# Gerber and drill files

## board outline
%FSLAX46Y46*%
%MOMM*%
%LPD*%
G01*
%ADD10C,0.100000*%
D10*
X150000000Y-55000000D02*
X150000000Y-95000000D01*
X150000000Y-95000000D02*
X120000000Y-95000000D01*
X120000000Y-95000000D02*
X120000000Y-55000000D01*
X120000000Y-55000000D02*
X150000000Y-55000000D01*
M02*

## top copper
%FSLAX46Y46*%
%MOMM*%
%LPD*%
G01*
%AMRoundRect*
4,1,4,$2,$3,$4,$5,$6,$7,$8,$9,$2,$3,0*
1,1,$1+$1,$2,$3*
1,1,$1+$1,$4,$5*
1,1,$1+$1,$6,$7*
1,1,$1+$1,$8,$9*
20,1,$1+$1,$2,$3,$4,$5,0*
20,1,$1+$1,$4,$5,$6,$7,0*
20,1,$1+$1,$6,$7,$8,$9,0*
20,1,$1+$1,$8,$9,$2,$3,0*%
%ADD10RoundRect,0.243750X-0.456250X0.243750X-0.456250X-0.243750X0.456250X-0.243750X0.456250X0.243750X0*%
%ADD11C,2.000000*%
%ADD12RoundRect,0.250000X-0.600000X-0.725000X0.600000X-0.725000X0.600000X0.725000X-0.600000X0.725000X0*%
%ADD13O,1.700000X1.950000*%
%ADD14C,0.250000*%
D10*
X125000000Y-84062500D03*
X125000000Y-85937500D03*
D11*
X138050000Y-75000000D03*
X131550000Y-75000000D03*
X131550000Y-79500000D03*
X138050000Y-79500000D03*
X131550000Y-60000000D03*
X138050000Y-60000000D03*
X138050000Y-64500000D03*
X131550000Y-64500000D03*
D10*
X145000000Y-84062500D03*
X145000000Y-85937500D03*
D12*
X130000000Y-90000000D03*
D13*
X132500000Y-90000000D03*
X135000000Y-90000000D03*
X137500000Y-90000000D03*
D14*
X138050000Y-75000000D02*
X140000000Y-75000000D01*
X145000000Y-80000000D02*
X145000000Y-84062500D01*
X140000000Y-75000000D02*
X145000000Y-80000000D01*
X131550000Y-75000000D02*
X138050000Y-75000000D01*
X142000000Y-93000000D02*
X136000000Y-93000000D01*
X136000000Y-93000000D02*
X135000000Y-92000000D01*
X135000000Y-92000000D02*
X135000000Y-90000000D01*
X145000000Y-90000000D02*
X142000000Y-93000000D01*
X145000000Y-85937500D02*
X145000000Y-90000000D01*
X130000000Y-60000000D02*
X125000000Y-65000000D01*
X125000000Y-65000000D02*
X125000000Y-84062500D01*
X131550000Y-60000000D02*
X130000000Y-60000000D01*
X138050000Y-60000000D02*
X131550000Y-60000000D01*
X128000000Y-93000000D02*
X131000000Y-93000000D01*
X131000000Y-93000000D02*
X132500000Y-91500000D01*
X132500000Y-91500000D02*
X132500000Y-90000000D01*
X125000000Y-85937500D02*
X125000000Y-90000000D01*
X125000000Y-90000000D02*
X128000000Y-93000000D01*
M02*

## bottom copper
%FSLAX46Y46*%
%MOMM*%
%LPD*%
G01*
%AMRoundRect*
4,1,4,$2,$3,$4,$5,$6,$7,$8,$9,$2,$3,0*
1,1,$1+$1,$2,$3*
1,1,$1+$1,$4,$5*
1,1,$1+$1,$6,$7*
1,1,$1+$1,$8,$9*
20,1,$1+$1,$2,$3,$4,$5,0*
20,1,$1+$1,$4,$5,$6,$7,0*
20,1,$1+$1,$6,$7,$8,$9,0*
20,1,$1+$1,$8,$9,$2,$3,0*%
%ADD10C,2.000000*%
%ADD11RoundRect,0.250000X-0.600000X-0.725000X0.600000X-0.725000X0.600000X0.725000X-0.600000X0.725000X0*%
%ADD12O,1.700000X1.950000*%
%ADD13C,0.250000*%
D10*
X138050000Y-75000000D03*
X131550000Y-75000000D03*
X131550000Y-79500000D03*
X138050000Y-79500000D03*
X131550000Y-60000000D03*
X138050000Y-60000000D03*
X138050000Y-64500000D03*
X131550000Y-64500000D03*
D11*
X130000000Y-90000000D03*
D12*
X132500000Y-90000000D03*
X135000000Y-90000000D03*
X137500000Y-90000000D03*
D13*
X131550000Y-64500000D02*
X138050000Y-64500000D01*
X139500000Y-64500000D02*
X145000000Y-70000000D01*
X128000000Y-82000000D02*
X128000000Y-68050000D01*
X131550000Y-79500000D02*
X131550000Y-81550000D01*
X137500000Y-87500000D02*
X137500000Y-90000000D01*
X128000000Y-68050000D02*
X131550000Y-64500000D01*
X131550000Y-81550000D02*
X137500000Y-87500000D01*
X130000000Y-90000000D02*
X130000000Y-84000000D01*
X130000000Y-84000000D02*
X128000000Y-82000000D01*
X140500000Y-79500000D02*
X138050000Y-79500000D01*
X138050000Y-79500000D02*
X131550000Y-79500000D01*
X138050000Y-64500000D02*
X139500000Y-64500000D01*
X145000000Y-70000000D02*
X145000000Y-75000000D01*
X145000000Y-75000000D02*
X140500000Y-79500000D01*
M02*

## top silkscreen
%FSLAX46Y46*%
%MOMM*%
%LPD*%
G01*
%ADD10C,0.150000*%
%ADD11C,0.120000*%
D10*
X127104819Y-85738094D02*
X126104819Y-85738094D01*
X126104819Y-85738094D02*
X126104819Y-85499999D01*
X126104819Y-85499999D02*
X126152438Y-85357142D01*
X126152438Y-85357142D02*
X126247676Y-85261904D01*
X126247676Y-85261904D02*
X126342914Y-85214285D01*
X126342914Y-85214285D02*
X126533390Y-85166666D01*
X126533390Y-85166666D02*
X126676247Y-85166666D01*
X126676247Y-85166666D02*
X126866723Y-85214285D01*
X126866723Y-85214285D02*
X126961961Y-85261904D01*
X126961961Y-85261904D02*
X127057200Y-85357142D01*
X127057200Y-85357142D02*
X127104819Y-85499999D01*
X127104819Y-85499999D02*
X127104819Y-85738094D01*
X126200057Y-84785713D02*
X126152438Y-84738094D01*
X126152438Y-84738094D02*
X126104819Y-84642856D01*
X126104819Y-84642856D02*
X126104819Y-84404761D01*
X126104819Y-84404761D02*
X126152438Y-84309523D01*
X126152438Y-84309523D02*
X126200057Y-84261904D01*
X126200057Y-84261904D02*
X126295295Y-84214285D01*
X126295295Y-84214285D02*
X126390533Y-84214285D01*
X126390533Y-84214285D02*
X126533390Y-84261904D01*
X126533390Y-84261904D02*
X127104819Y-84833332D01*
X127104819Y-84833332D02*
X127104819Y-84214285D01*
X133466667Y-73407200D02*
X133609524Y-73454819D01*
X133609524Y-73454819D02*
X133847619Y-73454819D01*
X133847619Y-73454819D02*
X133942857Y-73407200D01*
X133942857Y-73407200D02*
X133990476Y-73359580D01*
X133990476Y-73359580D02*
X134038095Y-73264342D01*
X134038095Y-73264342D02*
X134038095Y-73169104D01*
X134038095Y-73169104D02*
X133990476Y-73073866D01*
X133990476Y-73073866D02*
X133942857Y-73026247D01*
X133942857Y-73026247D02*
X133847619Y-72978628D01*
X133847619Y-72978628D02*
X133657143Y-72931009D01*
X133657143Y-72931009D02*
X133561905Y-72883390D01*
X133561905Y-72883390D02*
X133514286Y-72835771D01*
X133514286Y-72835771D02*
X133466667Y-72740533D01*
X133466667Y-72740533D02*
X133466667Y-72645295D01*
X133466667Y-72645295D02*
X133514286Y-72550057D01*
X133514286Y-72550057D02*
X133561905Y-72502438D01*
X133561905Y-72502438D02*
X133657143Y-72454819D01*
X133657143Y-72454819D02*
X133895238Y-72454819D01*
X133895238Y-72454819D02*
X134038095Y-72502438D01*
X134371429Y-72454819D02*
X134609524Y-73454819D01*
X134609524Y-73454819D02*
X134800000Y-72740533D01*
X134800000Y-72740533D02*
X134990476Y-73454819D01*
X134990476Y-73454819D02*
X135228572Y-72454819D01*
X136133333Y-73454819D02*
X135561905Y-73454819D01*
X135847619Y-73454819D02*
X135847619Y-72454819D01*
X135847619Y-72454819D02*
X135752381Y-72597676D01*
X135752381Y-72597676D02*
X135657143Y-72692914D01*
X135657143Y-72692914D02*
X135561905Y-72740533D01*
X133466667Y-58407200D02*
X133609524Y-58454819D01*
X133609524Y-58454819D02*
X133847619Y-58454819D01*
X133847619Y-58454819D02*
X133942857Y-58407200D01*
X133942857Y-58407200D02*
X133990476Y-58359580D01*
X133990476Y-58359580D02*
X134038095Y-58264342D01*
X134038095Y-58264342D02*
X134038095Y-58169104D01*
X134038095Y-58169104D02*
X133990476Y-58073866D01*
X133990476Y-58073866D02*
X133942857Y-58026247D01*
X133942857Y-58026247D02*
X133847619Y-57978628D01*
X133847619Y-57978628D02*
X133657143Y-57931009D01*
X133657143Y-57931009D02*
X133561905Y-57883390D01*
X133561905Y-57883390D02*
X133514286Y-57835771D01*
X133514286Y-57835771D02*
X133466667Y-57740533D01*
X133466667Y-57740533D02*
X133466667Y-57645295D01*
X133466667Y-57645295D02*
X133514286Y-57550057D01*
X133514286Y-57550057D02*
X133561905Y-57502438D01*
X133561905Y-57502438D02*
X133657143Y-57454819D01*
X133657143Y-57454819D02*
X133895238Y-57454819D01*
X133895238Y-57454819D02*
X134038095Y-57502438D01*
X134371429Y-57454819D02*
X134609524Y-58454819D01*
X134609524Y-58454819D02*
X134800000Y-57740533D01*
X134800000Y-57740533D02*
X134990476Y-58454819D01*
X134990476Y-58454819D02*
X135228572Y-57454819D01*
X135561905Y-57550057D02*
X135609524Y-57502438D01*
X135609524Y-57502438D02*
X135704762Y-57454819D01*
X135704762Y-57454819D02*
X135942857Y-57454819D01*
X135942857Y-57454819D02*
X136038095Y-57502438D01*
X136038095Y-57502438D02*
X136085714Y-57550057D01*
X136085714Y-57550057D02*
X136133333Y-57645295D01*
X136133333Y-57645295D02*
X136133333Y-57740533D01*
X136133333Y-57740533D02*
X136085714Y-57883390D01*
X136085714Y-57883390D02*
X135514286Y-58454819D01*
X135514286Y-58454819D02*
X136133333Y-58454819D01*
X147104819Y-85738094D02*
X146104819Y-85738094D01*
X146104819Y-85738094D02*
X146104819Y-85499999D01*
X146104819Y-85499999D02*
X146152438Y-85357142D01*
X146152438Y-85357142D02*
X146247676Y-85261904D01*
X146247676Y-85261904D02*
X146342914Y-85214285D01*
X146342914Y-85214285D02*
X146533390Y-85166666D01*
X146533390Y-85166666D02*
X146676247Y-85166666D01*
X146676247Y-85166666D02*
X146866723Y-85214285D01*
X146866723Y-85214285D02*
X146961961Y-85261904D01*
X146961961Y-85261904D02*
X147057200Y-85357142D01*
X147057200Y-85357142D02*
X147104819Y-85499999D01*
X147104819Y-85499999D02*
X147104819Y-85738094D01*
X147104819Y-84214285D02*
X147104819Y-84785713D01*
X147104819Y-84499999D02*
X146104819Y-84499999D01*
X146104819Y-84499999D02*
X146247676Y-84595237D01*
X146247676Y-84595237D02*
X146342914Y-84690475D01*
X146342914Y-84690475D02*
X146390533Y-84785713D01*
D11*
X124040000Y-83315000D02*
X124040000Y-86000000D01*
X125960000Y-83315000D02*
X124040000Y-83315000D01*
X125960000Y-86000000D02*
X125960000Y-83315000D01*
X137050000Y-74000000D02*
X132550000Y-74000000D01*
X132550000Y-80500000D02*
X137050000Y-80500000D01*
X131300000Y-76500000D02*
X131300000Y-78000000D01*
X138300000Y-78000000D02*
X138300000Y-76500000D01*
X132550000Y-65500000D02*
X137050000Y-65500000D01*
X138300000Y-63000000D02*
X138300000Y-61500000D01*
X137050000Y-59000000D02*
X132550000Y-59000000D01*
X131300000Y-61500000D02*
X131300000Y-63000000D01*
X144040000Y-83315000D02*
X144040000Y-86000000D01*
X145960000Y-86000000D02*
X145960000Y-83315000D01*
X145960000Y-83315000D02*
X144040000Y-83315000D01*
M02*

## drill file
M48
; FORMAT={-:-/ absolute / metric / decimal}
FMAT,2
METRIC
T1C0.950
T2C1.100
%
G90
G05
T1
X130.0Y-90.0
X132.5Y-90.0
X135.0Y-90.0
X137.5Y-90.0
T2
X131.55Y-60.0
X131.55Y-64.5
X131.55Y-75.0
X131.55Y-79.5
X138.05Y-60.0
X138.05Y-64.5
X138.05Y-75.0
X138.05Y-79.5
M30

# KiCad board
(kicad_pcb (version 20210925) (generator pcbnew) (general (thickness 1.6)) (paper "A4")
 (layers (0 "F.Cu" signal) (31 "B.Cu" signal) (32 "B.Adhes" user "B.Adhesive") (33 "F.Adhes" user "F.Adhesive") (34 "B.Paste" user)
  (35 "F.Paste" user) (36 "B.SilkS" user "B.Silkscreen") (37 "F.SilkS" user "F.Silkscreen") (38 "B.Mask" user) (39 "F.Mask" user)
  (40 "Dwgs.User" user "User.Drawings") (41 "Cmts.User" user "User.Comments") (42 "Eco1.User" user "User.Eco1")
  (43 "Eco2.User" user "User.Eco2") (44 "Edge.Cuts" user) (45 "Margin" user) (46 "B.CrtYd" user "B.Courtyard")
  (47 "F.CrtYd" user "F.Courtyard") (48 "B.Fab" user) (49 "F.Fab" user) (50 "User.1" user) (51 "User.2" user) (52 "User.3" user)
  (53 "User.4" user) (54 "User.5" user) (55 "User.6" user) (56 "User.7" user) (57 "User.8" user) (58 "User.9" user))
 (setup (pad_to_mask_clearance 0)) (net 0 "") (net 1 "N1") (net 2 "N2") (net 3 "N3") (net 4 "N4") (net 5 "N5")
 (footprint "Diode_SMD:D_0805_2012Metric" (layer "F.Cu") (at 125 85 -90)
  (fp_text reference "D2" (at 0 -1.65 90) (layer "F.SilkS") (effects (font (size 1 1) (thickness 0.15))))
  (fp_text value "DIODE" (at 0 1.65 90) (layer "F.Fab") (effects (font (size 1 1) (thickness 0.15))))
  (fp_line (start -1.685 0.96) (end 1 0.96) (layer "F.SilkS") (width 0.12))
  (fp_line (start -1.685 -0.96) (end -1.685 0.96) (layer "F.SilkS") (width 0.12))
  (fp_line (start 1 -0.96) (end -1.685 -0.96) (layer "F.SilkS") (width 0.12))
  (pad "1" smd roundrect locked (at -0.9375 0 270) (size 0.975 1.4) (layers "F.Cu" "F.Paste" "F.Mask") (roundrect_rratio 0.25) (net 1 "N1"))
  (pad "2" smd roundrect locked (at 0.9375 0 270) (size 0.975 1.4) (layers "F.Cu" "F.Paste" "F.Mask") (roundrect_rratio 0.25) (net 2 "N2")))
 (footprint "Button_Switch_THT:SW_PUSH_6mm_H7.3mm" (layer "F.Cu") (at 131.55 75)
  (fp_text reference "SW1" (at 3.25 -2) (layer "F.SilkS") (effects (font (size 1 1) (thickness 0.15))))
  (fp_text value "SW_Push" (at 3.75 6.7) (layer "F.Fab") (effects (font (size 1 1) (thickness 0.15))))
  (fp_line (start 5.5 -1) (end 1 -1) (layer "F.SilkS") (width 0.12))
  (fp_line (start 1 5.5) (end 5.5 5.5) (layer "F.SilkS") (width 0.12))
  (fp_line (start -0.25 1.5) (end -0.25 3) (layer "F.SilkS") (width 0.12))
  (fp_line (start 6.75 3) (end 6.75 1.5) (layer "F.SilkS") (width 0.12))
  (pad "1" thru_hole circle locked (at 6.5 0 90) (size 2 2) (drill 1.1) (layers *.Cu *.Mask) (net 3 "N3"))
  (pad "1" thru_hole circle locked (at 0 0 90) (size 2 2) (drill 1.1) (layers *.Cu *.Mask) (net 3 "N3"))
  (pad "2" thru_hole circle locked (at 0 4.5 90) (size 2 2) (drill 1.1) (layers *.Cu *.Mask) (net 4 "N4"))
  (pad "2" thru_hole circle locked (at 6.5 4.5 90) (size 2 2) (drill 1.1) (layers *.Cu *.Mask) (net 4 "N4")))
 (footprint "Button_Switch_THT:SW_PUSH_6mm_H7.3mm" (layer "F.Cu") (at 131.55 60)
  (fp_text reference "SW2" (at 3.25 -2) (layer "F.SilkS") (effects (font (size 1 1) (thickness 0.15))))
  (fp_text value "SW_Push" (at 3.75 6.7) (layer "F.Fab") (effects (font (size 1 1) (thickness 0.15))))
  (fp_line (start 1 5.5) (end 5.5 5.5) (layer "F.SilkS") (width 0.12))
  (fp_line (start 6.75 3) (end 6.75 1.5) (layer "F.SilkS") (width 0.12))
  (fp_line (start 5.5 -1) (end 1 -1) (layer "F.SilkS") (width 0.12))
  (fp_line (start -0.25 1.5) (end -0.25 3) (layer "F.SilkS") (width 0.12))
  (pad "1" thru_hole circle locked (at 0 0 90) (size 2 2) (drill 1.1) (layers *.Cu *.Mask) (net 1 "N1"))
  (pad "1" thru_hole circle locked (at 6.5 0 90) (size 2 2) (drill 1.1) (layers *.Cu *.Mask) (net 1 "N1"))
  (pad "2" thru_hole circle locked (at 6.5 4.5 90) (size 2 2) (drill 1.1) (layers *.Cu *.Mask) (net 4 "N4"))
  (pad "2" thru_hole circle locked (at 0 4.5 90) (size 2 2) (drill 1.1) (layers *.Cu *.Mask) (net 4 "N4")))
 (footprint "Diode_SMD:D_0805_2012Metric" (layer "F.Cu") (at 145 85 -90)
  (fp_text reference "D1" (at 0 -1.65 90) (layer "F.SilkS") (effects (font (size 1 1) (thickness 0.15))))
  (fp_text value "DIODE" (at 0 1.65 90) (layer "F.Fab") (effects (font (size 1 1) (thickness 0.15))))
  (fp_line (start -1.685 0.96) (end 1 0.96) (layer "F.SilkS") (width 0.12))
  (fp_line (start 1 -0.96) (end -1.685 -0.96) (layer "F.SilkS") (width 0.12))
  (fp_line (start -1.685 -0.96) (end -1.685 0.96) (layer "F.SilkS") (width 0.12))
  (pad "1" smd roundrect locked (at -0.9375 0 270) (size 0.975 1.4) (layers "F.Cu" "F.Paste" "F.Mask") (roundrect_rratio 0.25) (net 3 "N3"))
  (pad "2" smd roundrect locked (at 0.9375 0 270) (size 0.975 1.4) (layers "F.Cu" "F.Paste" "F.Mask") (roundrect_rratio 0.25) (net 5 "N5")))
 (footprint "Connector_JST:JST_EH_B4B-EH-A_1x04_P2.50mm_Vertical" (layer "B.Cu") (at 130 90)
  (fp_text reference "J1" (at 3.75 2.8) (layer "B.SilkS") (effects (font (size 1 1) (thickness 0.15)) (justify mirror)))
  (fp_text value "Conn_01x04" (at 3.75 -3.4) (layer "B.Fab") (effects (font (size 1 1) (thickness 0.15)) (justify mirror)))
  (pad "1" thru_hole roundrect locked (at 0 0) (size 1.7 1.95) (drill 0.95) (layers *.Cu *.Mask) (roundrect_rratio 0.147059) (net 4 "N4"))
  (pad "2" thru_hole oval locked (at 2.5 0) (size 1.7 1.95) (drill 0.95) (layers *.Cu *.Mask) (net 2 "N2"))
  (pad "3" thru_hole oval locked (at 5 0) (size 1.7 1.95) (drill 0.95) (layers *.Cu *.Mask) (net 5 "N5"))
  (pad "4" thru_hole oval locked (at 7.5 0) (size 1.7 1.95) (drill 0.95) (layers *.Cu *.Mask) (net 4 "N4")))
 (gr_line (start 150 55) (end 150 95) (layer "Edge.Cuts") (width 0.1))
 (gr_line (start 150 95) (end 120 95) (layer "Edge.Cuts") (width 0.1))
 (gr_line (start 120 95) (end 120 55) (layer "Edge.Cuts") (width 0.1))
 (gr_line (start 120 55) (end 150 55) (layer "Edge.Cuts") (width 0.1))
 (segment (start 138.05 75) (end 140 75) (width 0.25) (layer "F.Cu") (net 3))
 (segment (start 145 80) (end 145 84.0625) (width 0.25) (layer "F.Cu") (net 3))
 (segment (start 140 75) (end 145 80) (width 0.25) (layer "F.Cu") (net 3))
 (segment (start 131.55 75) (end 138.05 75) (width 0.25) (layer "F.Cu") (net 3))
 (segment (start 142 93) (end 136 93) (width 0.25) (layer "F.Cu") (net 5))
 (segment (start 136 93) (end 135 92) (width 0.25) (layer "F.Cu") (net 5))
 (segment (start 135 92) (end 135 90) (width 0.25) (layer "F.Cu") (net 5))
 (segment (start 145 90) (end 142 93) (width 0.25) (layer "F.Cu") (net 5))
 (segment (start 145 85.9375) (end 145 90) (width 0.25) (layer "F.Cu") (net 5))
 (segment (start 130 60) (end 125 65) (width 0.25) (layer "F.Cu") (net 1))
 (segment (start 125 65) (end 125 84.0625) (width 0.25) (layer "F.Cu") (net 1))
 (segment (start 131.55 60) (end 130 60) (width 0.25) (layer "F.Cu") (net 1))
 (segment (start 138.05 60) (end 131.55 60) (width 0.25) (layer "F.Cu") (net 1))
 (segment (start 128 93) (end 131 93) (width 0.25) (layer "F.Cu") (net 2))
 (segment (start 131 93) (end 132.5 91.5) (width 0.25) (layer "F.Cu") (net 2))
 (segment (start 132.5 91.5) (end 132.5 90) (width 0.25) (layer "F.Cu") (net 2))
 (segment (start 125 85.9375) (end 125 90) (width 0.25) (layer "F.Cu") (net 2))
 (segment (start 125 90) (end 128 93) (width 0.25) (layer "F.Cu") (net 2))
 (segment (start 131.55 64.5) (end 138.05 64.5) (width 0.25) (layer "B.Cu") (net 4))
 (segment (start 139.5 64.5) (end 145 70) (width 0.25) (layer "B.Cu") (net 4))
 (segment (start 128 82) (end 128 68.05) (width 0.25) (layer "B.Cu") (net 4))
 (segment (start 131.55 79.5) (end 131.55 81.55) (width 0.25) (layer "B.Cu") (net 4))
 (segment (start 137.5 87.5) (end 137.5 90) (width 0.25) (layer "B.Cu") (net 4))
 (segment (start 128 68.05) (end 131.55 64.5) (width 0.25) (layer "B.Cu") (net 4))
 (segment (start 131.55 81.55) (end 137.5 87.5) (width 0.25) (layer "B.Cu") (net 4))
 (segment (start 130 90) (end 130 84) (width 0.25) (layer "B.Cu") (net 4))
 (segment (start 130 84) (end 128 82) (width 0.25) (layer "B.Cu") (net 4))
 (segment (start 140.5 79.5) (end 138.05 79.5) (width 0.25) (layer "B.Cu") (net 4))
 (segment (start 138.05 79.5) (end 131.55 79.5) (width 0.25) (layer "B.Cu") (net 4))
 (segment (start 138.05 64.5) (end 139.5 64.5) (width 0.25) (layer "B.Cu") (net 4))
 (segment (start 145 70) (end 145 75) (width 0.25) (layer "B.Cu") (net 4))
 (segment (start 145 75) (end 140.5 79.5) (width 0.25) (layer "B.Cu") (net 4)))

